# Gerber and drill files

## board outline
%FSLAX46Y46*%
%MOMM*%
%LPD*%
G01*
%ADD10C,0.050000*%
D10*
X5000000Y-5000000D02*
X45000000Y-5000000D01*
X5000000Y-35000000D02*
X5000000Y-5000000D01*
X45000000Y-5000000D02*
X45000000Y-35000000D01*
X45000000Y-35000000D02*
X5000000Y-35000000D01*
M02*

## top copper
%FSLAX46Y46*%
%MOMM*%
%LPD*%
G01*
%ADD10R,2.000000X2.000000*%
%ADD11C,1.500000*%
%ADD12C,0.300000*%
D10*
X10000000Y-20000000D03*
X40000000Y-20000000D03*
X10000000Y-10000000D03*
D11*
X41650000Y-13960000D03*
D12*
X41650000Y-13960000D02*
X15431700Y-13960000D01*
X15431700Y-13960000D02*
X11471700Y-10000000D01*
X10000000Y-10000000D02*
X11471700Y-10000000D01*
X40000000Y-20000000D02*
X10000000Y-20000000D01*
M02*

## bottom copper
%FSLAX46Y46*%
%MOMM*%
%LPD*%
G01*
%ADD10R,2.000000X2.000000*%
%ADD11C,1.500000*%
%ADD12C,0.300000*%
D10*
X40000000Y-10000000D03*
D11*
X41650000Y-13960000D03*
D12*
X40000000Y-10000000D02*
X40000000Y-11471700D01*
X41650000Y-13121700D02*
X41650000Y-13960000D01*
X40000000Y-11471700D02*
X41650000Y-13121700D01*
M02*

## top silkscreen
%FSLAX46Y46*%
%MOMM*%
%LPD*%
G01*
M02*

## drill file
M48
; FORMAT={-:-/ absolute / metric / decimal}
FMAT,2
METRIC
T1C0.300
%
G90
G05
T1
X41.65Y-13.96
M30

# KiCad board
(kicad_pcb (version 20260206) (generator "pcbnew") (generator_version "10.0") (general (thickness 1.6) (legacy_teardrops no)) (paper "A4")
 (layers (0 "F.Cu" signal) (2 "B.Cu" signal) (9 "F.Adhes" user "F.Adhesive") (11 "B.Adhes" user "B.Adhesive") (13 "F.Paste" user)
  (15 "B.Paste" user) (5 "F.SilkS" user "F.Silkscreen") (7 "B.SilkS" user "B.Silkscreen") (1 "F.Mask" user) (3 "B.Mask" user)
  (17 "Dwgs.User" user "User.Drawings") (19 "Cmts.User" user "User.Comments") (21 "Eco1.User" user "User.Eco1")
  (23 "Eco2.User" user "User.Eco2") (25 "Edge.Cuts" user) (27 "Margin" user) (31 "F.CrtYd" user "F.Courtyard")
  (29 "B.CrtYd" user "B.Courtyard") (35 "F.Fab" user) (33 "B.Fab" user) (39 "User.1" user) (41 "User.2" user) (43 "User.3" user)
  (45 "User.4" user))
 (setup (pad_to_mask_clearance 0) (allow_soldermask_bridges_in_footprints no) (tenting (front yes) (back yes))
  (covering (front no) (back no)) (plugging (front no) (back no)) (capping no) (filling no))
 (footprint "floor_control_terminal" (layer "F.Cu") (at 10 20)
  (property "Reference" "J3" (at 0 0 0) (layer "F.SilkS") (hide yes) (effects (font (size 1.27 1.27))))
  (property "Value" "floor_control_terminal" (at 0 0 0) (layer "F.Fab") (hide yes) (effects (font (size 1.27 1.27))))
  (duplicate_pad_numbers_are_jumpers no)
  (pad "1" smd rect (at 0 0) (size 2 2) (layers "F.Cu" "F.Mask" "F.Paste") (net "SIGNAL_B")))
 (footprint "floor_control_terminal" (layer "F.Cu") (at 40 20)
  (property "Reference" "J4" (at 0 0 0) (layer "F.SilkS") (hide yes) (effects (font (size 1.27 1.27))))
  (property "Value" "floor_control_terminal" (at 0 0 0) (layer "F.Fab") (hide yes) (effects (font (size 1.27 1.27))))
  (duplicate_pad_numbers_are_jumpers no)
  (pad "1" smd rect (at 0 0) (size 2 2) (layers "F.Cu" "F.Mask" "F.Paste") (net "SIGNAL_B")))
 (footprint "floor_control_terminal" (layer "F.Cu") (at 10 10)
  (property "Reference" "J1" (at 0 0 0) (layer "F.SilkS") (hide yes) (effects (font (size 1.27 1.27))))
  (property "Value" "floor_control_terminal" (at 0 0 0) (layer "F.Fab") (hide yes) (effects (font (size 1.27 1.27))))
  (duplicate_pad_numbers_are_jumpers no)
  (pad "1" smd rect (at 0 0) (size 2 2) (layers "F.Cu" "F.Mask" "F.Paste") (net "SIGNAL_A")))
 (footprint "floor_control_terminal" (layer "B.Cu") (at 40 10)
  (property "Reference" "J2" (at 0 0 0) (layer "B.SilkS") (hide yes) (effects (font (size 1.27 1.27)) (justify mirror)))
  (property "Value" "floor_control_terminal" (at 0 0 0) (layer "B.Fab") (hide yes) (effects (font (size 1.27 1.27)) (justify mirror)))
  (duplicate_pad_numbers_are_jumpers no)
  (pad "1" smd rect (at 0 0) (size 2 2) (layers "B.Cu" "B.Mask" "B.Paste") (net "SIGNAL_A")))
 (gr_line (start 5 5) (end 45 5) (stroke (width 0.05) (type default)) (layer "Edge.Cuts"))
 (gr_line (start 5 35) (end 5 5) (stroke (width 0.05) (type default)) (layer "Edge.Cuts"))
 (gr_line (start 45 5) (end 45 35) (stroke (width 0.05) (type default)) (layer "Edge.Cuts"))
 (gr_line (start 45 35) (end 5 35) (stroke (width 0.05) (type default)) (layer "Edge.Cuts"))
 (segment (start 41.65 13.96) (end 15.4317 13.96) (width 0.3) (layer "F.Cu") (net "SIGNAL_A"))
 (segment (start 15.4317 13.96) (end 11.4717 10) (width 0.3) (layer "F.Cu") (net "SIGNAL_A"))
 (segment (start 10 10) (end 11.4717 10) (width 0.3) (layer "F.Cu") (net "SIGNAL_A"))
 (via (at 41.65 13.96) (size 1.5) (drill 0.3) (layers "F.Cu" "B.Cu") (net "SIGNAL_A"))
 (segment (start 40 10) (end 40 11.4717) (width 0.3) (layer "B.Cu") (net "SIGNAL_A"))
 (segment (start 41.65 13.1217) (end 41.65 13.96) (width 0.3) (layer "B.Cu") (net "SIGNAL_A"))
 (segment (start 40 11.4717) (end 41.65 13.1217) (width 0.3) (layer "B.Cu") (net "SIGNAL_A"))
 (segment (start 40 20) (end 10 20) (width 0.3) (layer "F.Cu") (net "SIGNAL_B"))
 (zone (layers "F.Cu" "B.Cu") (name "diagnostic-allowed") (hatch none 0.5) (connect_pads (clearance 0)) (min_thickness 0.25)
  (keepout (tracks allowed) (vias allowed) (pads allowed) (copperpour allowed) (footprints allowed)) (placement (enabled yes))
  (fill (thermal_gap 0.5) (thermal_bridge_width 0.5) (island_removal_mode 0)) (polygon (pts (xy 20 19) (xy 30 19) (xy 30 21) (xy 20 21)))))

